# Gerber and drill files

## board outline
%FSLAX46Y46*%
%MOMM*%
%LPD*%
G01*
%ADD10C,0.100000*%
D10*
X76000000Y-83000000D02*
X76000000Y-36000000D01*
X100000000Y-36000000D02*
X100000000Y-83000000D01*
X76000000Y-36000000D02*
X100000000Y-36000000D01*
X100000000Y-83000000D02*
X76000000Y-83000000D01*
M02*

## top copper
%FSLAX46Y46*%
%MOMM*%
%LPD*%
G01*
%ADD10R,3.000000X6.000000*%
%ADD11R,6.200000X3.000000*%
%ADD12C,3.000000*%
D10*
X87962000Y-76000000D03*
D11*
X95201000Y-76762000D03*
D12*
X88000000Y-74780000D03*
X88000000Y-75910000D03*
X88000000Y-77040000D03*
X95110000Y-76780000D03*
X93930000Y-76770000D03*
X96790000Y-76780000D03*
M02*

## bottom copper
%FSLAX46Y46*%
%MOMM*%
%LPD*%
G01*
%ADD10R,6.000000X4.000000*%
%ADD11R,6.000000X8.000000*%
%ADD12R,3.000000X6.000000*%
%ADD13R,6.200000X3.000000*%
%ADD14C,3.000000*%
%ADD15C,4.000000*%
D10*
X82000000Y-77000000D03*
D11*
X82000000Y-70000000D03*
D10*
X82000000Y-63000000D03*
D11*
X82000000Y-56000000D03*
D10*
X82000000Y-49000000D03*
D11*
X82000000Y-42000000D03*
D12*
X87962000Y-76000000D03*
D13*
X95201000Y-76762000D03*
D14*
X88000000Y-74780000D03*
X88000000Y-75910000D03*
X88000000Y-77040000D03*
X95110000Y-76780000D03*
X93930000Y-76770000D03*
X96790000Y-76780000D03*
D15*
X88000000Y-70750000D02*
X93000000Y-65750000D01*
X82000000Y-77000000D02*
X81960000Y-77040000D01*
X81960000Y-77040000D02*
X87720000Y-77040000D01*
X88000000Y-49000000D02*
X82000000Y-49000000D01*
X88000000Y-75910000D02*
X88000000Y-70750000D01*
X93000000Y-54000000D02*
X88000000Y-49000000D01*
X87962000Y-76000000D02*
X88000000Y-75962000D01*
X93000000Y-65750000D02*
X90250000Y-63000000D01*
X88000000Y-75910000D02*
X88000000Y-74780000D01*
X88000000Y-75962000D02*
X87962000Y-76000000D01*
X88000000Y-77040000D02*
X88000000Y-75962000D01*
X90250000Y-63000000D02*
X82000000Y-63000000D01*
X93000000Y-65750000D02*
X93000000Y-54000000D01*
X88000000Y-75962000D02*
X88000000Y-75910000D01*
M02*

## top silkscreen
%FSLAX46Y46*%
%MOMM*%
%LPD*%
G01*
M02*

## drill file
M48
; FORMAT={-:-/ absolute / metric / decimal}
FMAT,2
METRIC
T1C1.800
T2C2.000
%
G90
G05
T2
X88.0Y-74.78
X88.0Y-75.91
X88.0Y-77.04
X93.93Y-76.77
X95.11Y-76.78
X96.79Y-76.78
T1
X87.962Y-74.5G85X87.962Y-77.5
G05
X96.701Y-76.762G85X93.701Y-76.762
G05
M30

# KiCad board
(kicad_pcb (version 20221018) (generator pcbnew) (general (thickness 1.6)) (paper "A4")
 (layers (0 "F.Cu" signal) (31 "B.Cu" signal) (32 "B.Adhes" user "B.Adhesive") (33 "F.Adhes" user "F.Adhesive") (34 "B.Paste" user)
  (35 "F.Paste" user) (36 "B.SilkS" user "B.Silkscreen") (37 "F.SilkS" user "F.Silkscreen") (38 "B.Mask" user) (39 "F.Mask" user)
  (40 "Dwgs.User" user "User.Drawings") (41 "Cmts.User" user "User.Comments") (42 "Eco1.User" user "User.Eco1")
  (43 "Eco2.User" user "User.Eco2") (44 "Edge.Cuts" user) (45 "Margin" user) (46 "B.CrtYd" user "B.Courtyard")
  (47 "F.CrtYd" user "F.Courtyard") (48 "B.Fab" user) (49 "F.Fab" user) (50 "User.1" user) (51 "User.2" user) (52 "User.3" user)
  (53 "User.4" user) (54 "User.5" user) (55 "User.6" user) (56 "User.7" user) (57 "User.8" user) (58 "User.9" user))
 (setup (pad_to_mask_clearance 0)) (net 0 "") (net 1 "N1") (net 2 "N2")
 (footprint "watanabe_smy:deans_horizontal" (layer "B.Cu") (at 82 66 180)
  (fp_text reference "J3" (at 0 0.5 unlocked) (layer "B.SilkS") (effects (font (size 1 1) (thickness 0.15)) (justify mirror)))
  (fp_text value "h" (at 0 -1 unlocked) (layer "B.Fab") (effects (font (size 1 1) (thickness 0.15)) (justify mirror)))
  (pad "1" smd rect (at 0 -11) (size 6 4) (layers "B.Cu" "B.Paste" "B.Mask") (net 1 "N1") (thermal_bridge_angle 45))
  (pad "2" smd rect (at 0 -4 90) (size 8 6) (layers "B.Cu" "B.Paste" "B.Mask") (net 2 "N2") (thermal_bridge_angle 45)))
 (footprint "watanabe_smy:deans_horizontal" (layer "B.Cu") (at 82 52 180)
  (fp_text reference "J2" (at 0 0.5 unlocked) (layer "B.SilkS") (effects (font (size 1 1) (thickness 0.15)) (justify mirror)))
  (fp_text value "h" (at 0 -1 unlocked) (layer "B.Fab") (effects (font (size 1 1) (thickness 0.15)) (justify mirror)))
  (pad "1" smd rect (at 0 -11) (size 6 4) (layers "B.Cu" "B.Paste" "B.Mask") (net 1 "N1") (thermal_bridge_angle 45))
  (pad "2" smd rect (at 0 -4 90) (size 8 6) (layers "B.Cu" "B.Paste" "B.Mask") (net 2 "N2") (thermal_bridge_angle 45)))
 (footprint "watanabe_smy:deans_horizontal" (layer "B.Cu") (at 82 38 180)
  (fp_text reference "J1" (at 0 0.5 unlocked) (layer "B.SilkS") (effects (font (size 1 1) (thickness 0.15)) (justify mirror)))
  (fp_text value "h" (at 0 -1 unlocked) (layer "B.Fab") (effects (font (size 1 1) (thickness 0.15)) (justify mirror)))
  (pad "1" smd rect (at 0 -11) (size 6 4) (layers "B.Cu" "B.Paste" "B.Mask") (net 1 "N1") (thermal_bridge_angle 45))
  (pad "2" smd rect (at 0 -4 90) (size 8 6) (layers "B.Cu" "B.Paste" "B.Mask") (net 2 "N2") (thermal_bridge_angle 45)))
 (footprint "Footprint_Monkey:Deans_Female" (layer "B.Cu") (at 92.28 76 -90)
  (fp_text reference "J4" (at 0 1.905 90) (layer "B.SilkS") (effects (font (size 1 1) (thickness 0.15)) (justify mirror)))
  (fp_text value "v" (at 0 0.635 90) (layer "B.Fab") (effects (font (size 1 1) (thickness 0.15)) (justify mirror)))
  (pad "1" thru_hole rect (at 0 4.318 270) (size 6 3) (drill oval 4.8 1.8) (layers "*.Cu" "*.Mask") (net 1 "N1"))
  (pad "2" thru_hole rect (at 0.762 -2.921 180) (size 6.2 3) (drill oval 4.8 1.8) (layers "*.Cu" "*.Mask") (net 2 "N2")))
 (gr_line (start 76 83) (end 76 36) (stroke (width 0.1) (type default)) (layer "Edge.Cuts"))
 (gr_line (start 100 36) (end 100 83) (stroke (width 0.1) (type default)) (layer "Edge.Cuts"))
 (gr_line (start 76 36) (end 100 36) (stroke (width 0.1) (type default)) (layer "Edge.Cuts"))
 (gr_line (start 100 83) (end 76 83) (stroke (width 0.1) (type default)) (layer "Edge.Cuts"))
 (via (at 88 74.78) (size 3) (drill 2) (layers "F.Cu" "B.Cu") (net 1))
 (via (at 88 75.91) (size 3) (drill 2) (layers "F.Cu" "B.Cu") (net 1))
 (via (at 88 77.04) (size 3) (drill 2) (layers "F.Cu" "B.Cu") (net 1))
 (segment (start 88 70.75) (end 93 65.75) (width 4) (layer "B.Cu") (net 1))
 (segment (start 82 77) (end 81.96 77.04) (width 4) (layer "B.Cu") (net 1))
 (segment (start 81.96 77.04) (end 87.72 77.04) (width 4) (layer "B.Cu") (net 1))
 (segment (start 88 49) (end 82 49) (width 4) (layer "B.Cu") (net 1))
 (segment (start 88 75.91) (end 88 70.75) (width 4) (layer "B.Cu") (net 1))
 (segment (start 93 54) (end 88 49) (width 4) (layer "B.Cu") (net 1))
 (segment (start 87.962 76) (end 88 75.962) (width 4) (layer "B.Cu") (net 1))
 (segment (start 93 65.75) (end 90.25 63) (width 4) (layer "B.Cu") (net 1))
 (segment (start 88 75.91) (end 88 74.78) (width 4) (layer "B.Cu") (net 1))
 (segment (start 88 75.962) (end 87.962 76) (width 4) (layer "B.Cu") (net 1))
 (segment (start 88 77.04) (end 88 75.962) (width 4) (layer "B.Cu") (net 1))
 (segment (start 90.25 63) (end 82 63) (width 4) (layer "B.Cu") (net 1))
 (segment (start 93 65.75) (end 93 54) (width 4) (layer "B.Cu") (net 1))
 (segment (start 88 75.962) (end 88 75.91) (width 4) (layer "B.Cu") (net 1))
 (via (at 95.11 76.78) (size 3) (drill 2) (layers "F.Cu" "B.Cu") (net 2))
 (via (at 93.93 76.77) (size 3) (drill 2) (layers "F.Cu" "B.Cu") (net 2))
 (via (at 96.79 76.78) (size 3) (drill 2) (layers "F.Cu" "B.Cu") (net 2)))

